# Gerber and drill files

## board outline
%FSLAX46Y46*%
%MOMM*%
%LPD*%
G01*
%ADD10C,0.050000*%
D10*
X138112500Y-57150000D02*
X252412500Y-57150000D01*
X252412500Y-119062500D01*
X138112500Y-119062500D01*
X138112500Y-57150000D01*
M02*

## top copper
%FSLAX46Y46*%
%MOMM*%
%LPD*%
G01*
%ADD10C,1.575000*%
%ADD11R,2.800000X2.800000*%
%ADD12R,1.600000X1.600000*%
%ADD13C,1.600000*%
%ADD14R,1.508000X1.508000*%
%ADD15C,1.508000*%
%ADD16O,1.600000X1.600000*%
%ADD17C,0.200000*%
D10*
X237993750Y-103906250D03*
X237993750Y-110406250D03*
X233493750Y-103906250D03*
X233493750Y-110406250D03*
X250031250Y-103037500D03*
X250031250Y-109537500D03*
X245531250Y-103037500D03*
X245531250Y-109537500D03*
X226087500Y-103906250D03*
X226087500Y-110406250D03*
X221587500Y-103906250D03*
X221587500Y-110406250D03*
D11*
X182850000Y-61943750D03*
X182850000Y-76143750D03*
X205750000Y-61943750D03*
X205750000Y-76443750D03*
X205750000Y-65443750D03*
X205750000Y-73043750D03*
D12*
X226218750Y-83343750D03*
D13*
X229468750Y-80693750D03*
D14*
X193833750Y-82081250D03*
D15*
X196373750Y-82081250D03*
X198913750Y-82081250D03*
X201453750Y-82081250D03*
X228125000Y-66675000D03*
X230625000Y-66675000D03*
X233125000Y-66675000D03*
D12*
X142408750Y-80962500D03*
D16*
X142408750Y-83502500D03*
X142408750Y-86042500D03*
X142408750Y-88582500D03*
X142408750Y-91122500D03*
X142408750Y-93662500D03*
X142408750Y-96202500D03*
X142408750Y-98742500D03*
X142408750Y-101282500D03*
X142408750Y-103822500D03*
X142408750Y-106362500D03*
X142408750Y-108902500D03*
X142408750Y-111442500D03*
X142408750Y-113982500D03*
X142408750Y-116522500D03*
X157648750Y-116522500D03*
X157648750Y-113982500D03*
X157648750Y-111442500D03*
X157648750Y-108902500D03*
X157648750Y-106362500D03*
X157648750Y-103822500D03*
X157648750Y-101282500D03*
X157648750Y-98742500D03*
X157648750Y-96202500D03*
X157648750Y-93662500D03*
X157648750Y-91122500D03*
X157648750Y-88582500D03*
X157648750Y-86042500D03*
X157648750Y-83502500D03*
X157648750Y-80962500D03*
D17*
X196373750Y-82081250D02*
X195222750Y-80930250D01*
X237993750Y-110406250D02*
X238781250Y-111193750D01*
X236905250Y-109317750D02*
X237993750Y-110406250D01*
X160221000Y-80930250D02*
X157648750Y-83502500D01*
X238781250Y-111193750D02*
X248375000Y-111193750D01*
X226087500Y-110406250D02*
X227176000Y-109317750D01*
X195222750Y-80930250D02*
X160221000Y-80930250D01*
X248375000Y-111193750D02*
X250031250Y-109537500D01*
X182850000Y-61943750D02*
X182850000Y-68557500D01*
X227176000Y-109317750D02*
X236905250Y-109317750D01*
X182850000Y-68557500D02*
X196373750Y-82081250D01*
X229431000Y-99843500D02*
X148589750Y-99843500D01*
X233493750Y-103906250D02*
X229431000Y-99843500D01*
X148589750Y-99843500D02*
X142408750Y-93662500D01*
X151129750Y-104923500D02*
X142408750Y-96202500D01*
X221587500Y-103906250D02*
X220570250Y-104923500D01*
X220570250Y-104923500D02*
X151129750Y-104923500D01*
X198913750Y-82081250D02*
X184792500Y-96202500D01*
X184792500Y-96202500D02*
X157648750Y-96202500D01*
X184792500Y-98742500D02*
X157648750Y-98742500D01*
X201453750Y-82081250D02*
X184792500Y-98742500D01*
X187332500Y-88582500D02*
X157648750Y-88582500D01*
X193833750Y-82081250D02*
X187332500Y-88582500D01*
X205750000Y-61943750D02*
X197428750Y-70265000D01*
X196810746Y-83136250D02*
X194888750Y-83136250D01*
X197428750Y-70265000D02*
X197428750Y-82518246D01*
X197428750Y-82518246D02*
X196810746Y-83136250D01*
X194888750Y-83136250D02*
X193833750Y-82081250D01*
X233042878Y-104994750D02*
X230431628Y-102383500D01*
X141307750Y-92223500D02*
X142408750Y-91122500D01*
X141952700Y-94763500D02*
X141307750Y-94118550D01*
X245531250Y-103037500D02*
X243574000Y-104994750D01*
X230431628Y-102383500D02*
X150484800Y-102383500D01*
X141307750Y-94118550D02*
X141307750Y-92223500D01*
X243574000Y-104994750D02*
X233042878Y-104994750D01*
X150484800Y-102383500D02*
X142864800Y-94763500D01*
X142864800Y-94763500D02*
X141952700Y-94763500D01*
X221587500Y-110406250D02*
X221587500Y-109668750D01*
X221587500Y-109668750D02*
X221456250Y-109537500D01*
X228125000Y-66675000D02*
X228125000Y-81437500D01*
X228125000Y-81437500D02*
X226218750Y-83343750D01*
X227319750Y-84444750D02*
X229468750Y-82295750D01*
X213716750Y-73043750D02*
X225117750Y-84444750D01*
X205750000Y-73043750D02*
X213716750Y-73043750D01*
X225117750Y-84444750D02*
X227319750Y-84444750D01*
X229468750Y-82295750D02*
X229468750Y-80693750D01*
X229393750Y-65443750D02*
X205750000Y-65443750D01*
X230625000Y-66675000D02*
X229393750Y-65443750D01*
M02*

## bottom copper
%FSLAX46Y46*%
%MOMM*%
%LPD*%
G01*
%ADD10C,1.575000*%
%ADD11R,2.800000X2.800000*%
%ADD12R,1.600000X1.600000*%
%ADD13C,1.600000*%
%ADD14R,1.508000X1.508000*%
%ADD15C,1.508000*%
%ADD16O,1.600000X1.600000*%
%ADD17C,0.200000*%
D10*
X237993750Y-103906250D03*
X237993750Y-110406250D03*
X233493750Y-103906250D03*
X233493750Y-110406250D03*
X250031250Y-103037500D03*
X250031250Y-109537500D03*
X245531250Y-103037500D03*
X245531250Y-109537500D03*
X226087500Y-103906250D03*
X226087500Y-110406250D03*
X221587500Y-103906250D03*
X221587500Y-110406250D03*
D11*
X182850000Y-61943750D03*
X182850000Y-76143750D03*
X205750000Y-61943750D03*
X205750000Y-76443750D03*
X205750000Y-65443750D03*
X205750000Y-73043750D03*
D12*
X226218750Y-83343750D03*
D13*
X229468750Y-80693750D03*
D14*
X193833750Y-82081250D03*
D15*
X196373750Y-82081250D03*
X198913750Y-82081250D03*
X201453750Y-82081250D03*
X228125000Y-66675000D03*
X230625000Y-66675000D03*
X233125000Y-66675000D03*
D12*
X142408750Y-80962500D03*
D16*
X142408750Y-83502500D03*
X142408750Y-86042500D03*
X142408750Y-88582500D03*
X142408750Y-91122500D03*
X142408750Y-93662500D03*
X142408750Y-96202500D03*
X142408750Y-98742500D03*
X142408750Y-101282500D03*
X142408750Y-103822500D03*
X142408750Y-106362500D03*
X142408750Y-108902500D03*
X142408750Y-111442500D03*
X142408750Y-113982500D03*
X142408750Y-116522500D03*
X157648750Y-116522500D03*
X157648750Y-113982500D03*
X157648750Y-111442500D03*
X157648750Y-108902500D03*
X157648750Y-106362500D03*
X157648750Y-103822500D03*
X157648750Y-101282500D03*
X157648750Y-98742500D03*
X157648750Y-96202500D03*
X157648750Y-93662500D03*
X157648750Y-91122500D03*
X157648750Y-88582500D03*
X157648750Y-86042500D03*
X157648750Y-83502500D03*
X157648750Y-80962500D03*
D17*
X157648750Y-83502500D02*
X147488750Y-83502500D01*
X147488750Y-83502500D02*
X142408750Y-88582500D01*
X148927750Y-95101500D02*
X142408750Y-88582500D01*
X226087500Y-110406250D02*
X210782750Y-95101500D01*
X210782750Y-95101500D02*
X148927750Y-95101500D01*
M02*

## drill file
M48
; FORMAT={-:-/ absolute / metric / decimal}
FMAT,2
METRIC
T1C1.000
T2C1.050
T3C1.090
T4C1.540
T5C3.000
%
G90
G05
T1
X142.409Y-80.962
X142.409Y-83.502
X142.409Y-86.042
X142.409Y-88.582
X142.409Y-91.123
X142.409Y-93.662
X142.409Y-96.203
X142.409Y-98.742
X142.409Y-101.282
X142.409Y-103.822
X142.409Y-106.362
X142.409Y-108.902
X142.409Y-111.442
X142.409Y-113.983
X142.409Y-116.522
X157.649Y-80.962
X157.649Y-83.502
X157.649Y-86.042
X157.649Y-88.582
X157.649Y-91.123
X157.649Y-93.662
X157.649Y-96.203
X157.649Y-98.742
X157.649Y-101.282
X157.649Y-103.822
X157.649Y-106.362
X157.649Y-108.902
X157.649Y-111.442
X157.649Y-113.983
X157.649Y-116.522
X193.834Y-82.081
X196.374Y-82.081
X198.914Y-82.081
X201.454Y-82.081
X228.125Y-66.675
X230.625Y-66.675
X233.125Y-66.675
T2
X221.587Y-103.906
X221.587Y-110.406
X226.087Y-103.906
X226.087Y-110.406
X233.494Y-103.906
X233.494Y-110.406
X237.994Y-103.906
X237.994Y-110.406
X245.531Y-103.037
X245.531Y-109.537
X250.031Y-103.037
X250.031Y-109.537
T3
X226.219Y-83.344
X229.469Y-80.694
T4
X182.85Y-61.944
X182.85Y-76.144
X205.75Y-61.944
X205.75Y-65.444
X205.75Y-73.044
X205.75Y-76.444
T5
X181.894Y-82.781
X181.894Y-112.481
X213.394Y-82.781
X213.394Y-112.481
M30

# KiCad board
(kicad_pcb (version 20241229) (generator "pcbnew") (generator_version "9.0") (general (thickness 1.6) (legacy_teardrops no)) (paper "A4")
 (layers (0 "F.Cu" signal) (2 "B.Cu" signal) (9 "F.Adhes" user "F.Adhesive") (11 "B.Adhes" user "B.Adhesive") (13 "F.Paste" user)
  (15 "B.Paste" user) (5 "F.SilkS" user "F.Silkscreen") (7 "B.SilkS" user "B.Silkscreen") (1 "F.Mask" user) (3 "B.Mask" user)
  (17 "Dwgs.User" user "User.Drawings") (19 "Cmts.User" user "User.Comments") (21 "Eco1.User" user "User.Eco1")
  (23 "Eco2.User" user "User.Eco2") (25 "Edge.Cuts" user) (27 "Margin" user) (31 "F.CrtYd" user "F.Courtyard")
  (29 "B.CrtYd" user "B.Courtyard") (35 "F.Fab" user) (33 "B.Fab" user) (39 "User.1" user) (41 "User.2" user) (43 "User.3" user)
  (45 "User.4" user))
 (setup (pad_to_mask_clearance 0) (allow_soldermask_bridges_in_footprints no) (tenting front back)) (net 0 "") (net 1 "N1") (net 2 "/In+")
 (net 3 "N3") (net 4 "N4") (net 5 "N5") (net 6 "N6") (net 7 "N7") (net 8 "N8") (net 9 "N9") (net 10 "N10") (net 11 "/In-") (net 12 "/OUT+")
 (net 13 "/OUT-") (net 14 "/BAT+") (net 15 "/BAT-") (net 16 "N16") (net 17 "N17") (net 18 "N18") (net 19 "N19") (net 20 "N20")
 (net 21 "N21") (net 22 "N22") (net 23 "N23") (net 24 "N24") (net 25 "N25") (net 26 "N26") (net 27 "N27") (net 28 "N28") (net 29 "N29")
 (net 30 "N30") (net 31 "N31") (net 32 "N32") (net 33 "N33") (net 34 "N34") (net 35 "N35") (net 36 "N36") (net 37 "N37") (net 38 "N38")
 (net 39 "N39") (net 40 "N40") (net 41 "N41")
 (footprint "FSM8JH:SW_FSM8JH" (layer "F.Cu") (at 235.74375 107.15625)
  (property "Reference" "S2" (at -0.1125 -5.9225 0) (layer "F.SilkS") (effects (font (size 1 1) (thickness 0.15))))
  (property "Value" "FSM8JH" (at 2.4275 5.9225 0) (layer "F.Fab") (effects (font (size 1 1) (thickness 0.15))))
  (pad "1" thru_hole circle (at 2.25 -3.25) (size 1.575 1.575) (drill 1.05) (layers "*.Cu" "*.Mask") (remove_unused_layers no) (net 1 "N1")
   (solder_mask_margin 0.102))
  (pad "2" thru_hole circle (at 2.25 3.25) (size 1.575 1.575) (drill 1.05) (layers "*.Cu" "*.Mask") (remove_unused_layers no) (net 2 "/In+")
   (solder_mask_margin 0.102))
  (pad "3" thru_hole circle (at -2.25 -3.25) (size 1.575 1.575) (drill 1.05) (layers "*.Cu" "*.Mask") (remove_unused_layers no) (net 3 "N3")
   (solder_mask_margin 0.102))
  (pad "4" thru_hole circle (at -2.25 3.25) (size 1.575 1.575) (drill 1.05) (layers "*.Cu" "*.Mask") (remove_unused_layers no) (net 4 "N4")
   (solder_mask_margin 0.102)))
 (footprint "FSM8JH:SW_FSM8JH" (layer "F.Cu") (at 247.78125 106.2875)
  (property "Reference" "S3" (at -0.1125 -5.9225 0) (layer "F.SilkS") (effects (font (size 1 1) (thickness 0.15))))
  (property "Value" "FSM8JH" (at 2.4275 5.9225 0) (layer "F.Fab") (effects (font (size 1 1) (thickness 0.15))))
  (pad "1" thru_hole circle (at 2.25 -3.25) (size 1.575 1.575) (drill 1.05) (layers "*.Cu" "*.Mask") (remove_unused_layers no) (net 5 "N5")
   (solder_mask_margin 0.102))
  (pad "2" thru_hole circle (at 2.25 3.25) (size 1.575 1.575) (drill 1.05) (layers "*.Cu" "*.Mask") (remove_unused_layers no) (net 2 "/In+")
   (solder_mask_margin 0.102))
  (pad "3" thru_hole circle (at -2.25 -3.25) (size 1.575 1.575) (drill 1.05) (layers "*.Cu" "*.Mask") (remove_unused_layers no) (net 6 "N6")
   (solder_mask_margin 0.102))
  (pad "4" thru_hole circle (at -2.25 3.25) (size 1.575 1.575) (drill 1.05) (layers "*.Cu" "*.Mask") (remove_unused_layers no) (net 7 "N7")
   (solder_mask_margin 0.102)))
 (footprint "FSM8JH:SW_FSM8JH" (layer "F.Cu") (at 223.8375 107.15625)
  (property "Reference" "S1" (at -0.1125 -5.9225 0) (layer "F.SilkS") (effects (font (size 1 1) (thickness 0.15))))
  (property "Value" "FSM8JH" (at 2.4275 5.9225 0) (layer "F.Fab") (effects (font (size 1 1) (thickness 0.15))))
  (pad "1" thru_hole circle (at 2.25 -3.25) (size 1.575 1.575) (drill 1.05) (layers "*.Cu" "*.Mask") (remove_unused_layers no) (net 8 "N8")
   (solder_mask_margin 0.102))
  (pad "2" thru_hole circle (at 2.25 3.25) (size 1.575 1.575) (drill 1.05) (layers "*.Cu" "*.Mask") (remove_unused_layers no) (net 2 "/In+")
   (solder_mask_margin 0.102))
  (pad "3" thru_hole circle (at -2.25 -3.25) (size 1.575 1.575) (drill 1.05) (layers "*.Cu" "*.Mask") (remove_unused_layers no) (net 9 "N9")
   (solder_mask_margin 0.102))
  (pad "4" thru_hole circle (at -2.25 3.25) (size 1.575 1.575) (drill 1.05) (layers "*.Cu" "*.Mask") (remove_unused_layers no)
   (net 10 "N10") (solder_mask_margin 0.102)))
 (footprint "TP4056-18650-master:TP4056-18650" (layer "F.Cu") (at 181.15 60.24375)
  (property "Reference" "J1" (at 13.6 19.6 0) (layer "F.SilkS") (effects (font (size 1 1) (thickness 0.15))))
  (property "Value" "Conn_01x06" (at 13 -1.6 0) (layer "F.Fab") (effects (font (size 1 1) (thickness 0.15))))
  (pad "1" thru_hole rect (at 1.7 1.7) (size 2.8 2.8) (drill 1.54) (layers "*.Cu" "*.Mask") (remove_unused_layers no) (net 2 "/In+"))
  (pad "2" thru_hole rect (at 1.7 15.9) (size 2.8 2.8) (drill 1.54) (layers "*.Cu" "*.Mask") (remove_unused_layers no) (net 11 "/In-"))
  (pad "3" thru_hole rect (at 24.6 1.7) (size 2.8 2.8) (drill 1.54) (layers "*.Cu" "*.Mask") (remove_unused_layers no) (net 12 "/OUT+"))
  (pad "4" thru_hole rect (at 24.6 16.2) (size 2.8 2.8) (drill 1.54) (layers "*.Cu" "*.Mask") (remove_unused_layers no) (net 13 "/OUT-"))
  (pad "5" thru_hole rect (at 24.6 5.2) (size 2.8 2.8) (drill 1.54) (layers "*.Cu" "*.Mask") (remove_unused_layers no) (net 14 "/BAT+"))
  (pad "6" thru_hole rect (at 24.6 12.8) (size 2.8 2.8) (drill 1.54) (layers "*.Cu" "*.Mask") (remove_unused_layers no) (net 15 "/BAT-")))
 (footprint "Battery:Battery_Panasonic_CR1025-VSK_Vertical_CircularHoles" (layer "F.Cu") (at 226.21875 83.34375)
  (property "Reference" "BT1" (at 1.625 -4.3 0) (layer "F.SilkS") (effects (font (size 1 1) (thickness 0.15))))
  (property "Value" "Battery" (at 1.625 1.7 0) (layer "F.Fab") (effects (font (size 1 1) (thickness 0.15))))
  (pad "1" thru_hole rect (at 0 0) (size 1.6 1.6) (drill 1.09) (layers "*.Cu" "*.Mask") (remove_unused_layers no) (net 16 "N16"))
  (pad "2" thru_hole circle (at 3.25 -2.65) (size 1.6 1.6) (drill 1.09) (layers "*.Cu" "*.Mask") (remove_unused_layers no) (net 15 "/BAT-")))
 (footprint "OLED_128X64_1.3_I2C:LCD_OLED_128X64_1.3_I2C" (layer "F.Cu") (at 197.64375 97.63125)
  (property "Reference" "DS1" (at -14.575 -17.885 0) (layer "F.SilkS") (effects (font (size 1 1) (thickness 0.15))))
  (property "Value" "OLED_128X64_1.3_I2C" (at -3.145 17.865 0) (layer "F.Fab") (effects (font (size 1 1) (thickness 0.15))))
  (pad "" np_thru_hole circle (at -15.75 -14.85) (size 3 3) (drill 3) (layers "*.Cu" "*.Mask"))
  (pad "" np_thru_hole circle (at -15.75 14.85) (size 3 3) (drill 3) (layers "*.Cu" "*.Mask"))
  (pad "" np_thru_hole circle (at 15.75 -14.85) (size 3 3) (drill 3) (layers "*.Cu" "*.Mask"))
  (pad "" np_thru_hole circle (at 15.75 14.85) (size 3 3) (drill 3) (layers "*.Cu" "*.Mask"))
  (pad "1" thru_hole rect (at -3.81 -15.55) (size 1.508 1.508) (drill 1) (layers "*.Cu" "*.Mask") (remove_unused_layers no) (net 12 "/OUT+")
   (solder_mask_margin 0.102))
  (pad "2" thru_hole circle (at -1.27 -15.55) (size 1.508 1.508) (drill 1) (layers "*.Cu" "*.Mask") (remove_unused_layers no) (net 2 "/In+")
   (solder_mask_margin 0.102))
  (pad "3" thru_hole circle (at 1.27 -15.55) (size 1.508 1.508) (drill 1) (layers "*.Cu" "*.Mask") (remove_unused_layers no) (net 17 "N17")
   (solder_mask_margin 0.102))
  (pad "4" thru_hole circle (at 3.81 -15.55) (size 1.508 1.508) (drill 1) (layers "*.Cu" "*.Mask") (remove_unused_layers no) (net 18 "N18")
   (solder_mask_margin 0.102)))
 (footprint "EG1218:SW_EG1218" (layer "F.Cu") (at 230.625 66.675)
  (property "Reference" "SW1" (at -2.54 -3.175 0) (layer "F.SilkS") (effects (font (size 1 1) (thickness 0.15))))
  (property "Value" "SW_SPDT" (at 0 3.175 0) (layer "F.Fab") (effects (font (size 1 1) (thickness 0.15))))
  (pad "1" thru_hole circle (at -2.5 0) (size 1.508 1.508) (drill 1) (layers "*.Cu" "*.Mask") (remove_unused_layers no) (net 16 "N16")
   (solder_mask_margin 0.102))
  (pad "2" thru_hole circle (at 0 0) (size 1.508 1.508) (drill 1) (layers "*.Cu" "*.Mask") (remove_unused_layers no) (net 14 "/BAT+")
   (solder_mask_margin 0.102))
  (pad "3" thru_hole circle (at 2.5 0) (size 1.508 1.508) (drill 1) (layers "*.Cu" "*.Mask") (remove_unused_layers no) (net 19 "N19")
   (solder_mask_margin 0.102)))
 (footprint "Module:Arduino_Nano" (layer "F.Cu") (at 142.40875 80.9625)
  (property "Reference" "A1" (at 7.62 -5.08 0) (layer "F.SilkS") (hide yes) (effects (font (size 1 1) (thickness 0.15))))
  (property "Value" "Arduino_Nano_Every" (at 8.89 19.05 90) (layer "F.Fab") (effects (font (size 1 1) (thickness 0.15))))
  (pad "1" thru_hole rect (at 0 0) (size 1.6 1.6) (drill 1) (layers "*.Cu" "*.Mask") (remove_unused_layers no) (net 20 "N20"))
  (pad "2" thru_hole oval (at 0 2.54) (size 1.6 1.6) (drill 1) (layers "*.Cu" "*.Mask") (remove_unused_layers no) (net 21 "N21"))
  (pad "3" thru_hole oval (at 0 5.08) (size 1.6 1.6) (drill 1) (layers "*.Cu" "*.Mask") (remove_unused_layers no) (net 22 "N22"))
  (pad "4" thru_hole oval (at 0 7.62) (size 1.6 1.6) (drill 1) (layers "*.Cu" "*.Mask") (remove_unused_layers no) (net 2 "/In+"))
  (pad "5" thru_hole oval (at 0 10.16) (size 1.6 1.6) (drill 1) (layers "*.Cu" "*.Mask") (remove_unused_layers no) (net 6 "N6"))
  (pad "6" thru_hole oval (at 0 12.7) (size 1.6 1.6) (drill 1) (layers "*.Cu" "*.Mask") (remove_unused_layers no) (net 3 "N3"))
  (pad "7" thru_hole oval (at 0 15.24) (size 1.6 1.6) (drill 1) (layers "*.Cu" "*.Mask") (remove_unused_layers no) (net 9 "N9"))
  (pad "8" thru_hole oval (at 0 17.78) (size 1.6 1.6) (drill 1) (layers "*.Cu" "*.Mask") (remove_unused_layers no) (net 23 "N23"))
  (pad "9" thru_hole oval (at 0 20.32) (size 1.6 1.6) (drill 1) (layers "*.Cu" "*.Mask") (remove_unused_layers no) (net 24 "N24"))
  (pad "10" thru_hole oval (at 0 22.86) (size 1.6 1.6) (drill 1) (layers "*.Cu" "*.Mask") (remove_unused_layers no) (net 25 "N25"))
  (pad "11" thru_hole oval (at 0 25.4) (size 1.6 1.6) (drill 1) (layers "*.Cu" "*.Mask") (remove_unused_layers no) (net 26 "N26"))
  (pad "12" thru_hole oval (at 0 27.94) (size 1.6 1.6) (drill 1) (layers "*.Cu" "*.Mask") (remove_unused_layers no) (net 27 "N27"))
  (pad "13" thru_hole oval (at 0 30.48) (size 1.6 1.6) (drill 1) (layers "*.Cu" "*.Mask") (remove_unused_layers no) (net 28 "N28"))
  (pad "14" thru_hole oval (at 0 33.02) (size 1.6 1.6) (drill 1) (layers "*.Cu" "*.Mask") (remove_unused_layers no) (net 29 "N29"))
  (pad "15" thru_hole oval (at 0 35.56) (size 1.6 1.6) (drill 1) (layers "*.Cu" "*.Mask") (remove_unused_layers no) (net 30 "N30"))
  (pad "16" thru_hole oval (at 15.24 35.56) (size 1.6 1.6) (drill 1) (layers "*.Cu" "*.Mask") (remove_unused_layers no) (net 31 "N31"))
  (pad "17" thru_hole oval (at 15.24 33.02) (size 1.6 1.6) (drill 1) (layers "*.Cu" "*.Mask") (remove_unused_layers no) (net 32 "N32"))
  (pad "18" thru_hole oval (at 15.24 30.48) (size 1.6 1.6) (drill 1) (layers "*.Cu" "*.Mask") (remove_unused_layers no) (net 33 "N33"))
  (pad "19" thru_hole oval (at 15.24 27.94) (size 1.6 1.6) (drill 1) (layers "*.Cu" "*.Mask") (remove_unused_layers no) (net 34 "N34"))
  (pad "20" thru_hole oval (at 15.24 25.4) (size 1.6 1.6) (drill 1) (layers "*.Cu" "*.Mask") (remove_unused_layers no) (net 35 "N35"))
  (pad "21" thru_hole oval (at 15.24 22.86) (size 1.6 1.6) (drill 1) (layers "*.Cu" "*.Mask") (remove_unused_layers no) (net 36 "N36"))
  (pad "22" thru_hole oval (at 15.24 20.32) (size 1.6 1.6) (drill 1) (layers "*.Cu" "*.Mask") (remove_unused_layers no) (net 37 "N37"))
  (pad "23" thru_hole oval (at 15.24 17.78) (size 1.6 1.6) (drill 1) (layers "*.Cu" "*.Mask") (remove_unused_layers no) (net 18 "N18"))
  (pad "24" thru_hole oval (at 15.24 15.24) (size 1.6 1.6) (drill 1) (layers "*.Cu" "*.Mask") (remove_unused_layers no) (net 17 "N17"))
  (pad "25" thru_hole oval (at 15.24 12.7) (size 1.6 1.6) (drill 1) (layers "*.Cu" "*.Mask") (remove_unused_layers no) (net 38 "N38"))
  (pad "26" thru_hole oval (at 15.24 10.16) (size 1.6 1.6) (drill 1) (layers "*.Cu" "*.Mask") (remove_unused_layers no) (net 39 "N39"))
  (pad "27" thru_hole oval (at 15.24 7.62) (size 1.6 1.6) (drill 1) (layers "*.Cu" "*.Mask") (remove_unused_layers no) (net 12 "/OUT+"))
  (pad "28" thru_hole oval (at 15.24 5.08) (size 1.6 1.6) (drill 1) (layers "*.Cu" "*.Mask") (remove_unused_layers no) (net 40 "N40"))
  (pad "29" thru_hole oval (at 15.24 2.54) (size 1.6 1.6) (drill 1) (layers "*.Cu" "*.Mask") (remove_unused_layers no) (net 2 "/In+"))
  (pad "30" thru_hole oval (at 15.24 0) (size 1.6 1.6) (drill 1) (layers "*.Cu" "*.Mask") (remove_unused_layers no) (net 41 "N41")))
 (gr_rect (start 138.1125 57.15) (end 252.4125 119.0625) (stroke (width 0.05) (type default)) (fill no) (layer "Edge.Cuts"))
 (segment (start 196.37375 82.08125) (end 195.22275 80.93025) (width 0.2) (layer "F.Cu") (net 2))
 (segment (start 237.99375 110.40625) (end 238.78125 111.19375) (width 0.2) (layer "F.Cu") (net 2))
 (segment (start 236.90525 109.31775) (end 237.99375 110.40625) (width 0.2) (layer "F.Cu") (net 2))
 (segment (start 160.221 80.93025) (end 157.64875 83.5025) (width 0.2) (layer "F.Cu") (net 2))
 (segment (start 238.78125 111.19375) (end 248.375 111.19375) (width 0.2) (layer "F.Cu") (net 2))
 (segment (start 226.0875 110.40625) (end 227.176 109.31775) (width 0.2) (layer "F.Cu") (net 2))
 (segment (start 195.22275 80.93025) (end 160.221 80.93025) (width 0.2) (layer "F.Cu") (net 2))
 (segment (start 248.375 111.19375) (end 250.03125 109.5375) (width 0.2) (layer "F.Cu") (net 2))
 (segment (start 182.85 61.94375) (end 182.85 68.5575) (width 0.2) (layer "F.Cu") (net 2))
 (segment (start 227.176 109.31775) (end 236.90525 109.31775) (width 0.2) (layer "F.Cu") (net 2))
 (segment (start 182.85 68.5575) (end 196.37375 82.08125) (width 0.2) (layer "F.Cu") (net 2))
 (segment (start 157.64875 83.5025) (end 147.48875 83.5025) (width 0.2) (layer "B.Cu") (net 2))
 (segment (start 147.48875 83.5025) (end 142.40875 88.5825) (width 0.2) (layer "B.Cu") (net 2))
 (segment (start 148.92775 95.1015) (end 142.40875 88.5825) (width 0.2) (layer "B.Cu") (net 2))
 (segment (start 226.0875 110.40625) (end 210.78275 95.1015) (width 0.2) (layer "B.Cu") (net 2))
 (segment (start 210.78275 95.1015) (end 148.92775 95.1015) (width 0.2) (layer "B.Cu") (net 2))
 (segment (start 229.431 99.8435) (end 148.58975 99.8435) (width 0.2) (layer "F.Cu") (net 3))
 (segment (start 233.49375 103.90625) (end 229.431 99.8435) (width 0.2) (layer "F.Cu") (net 3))
 (segment (start 148.58975 99.8435) (end 142.40875 93.6625) (width 0.2) (layer "F.Cu") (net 3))
 (segment (start 151.12975 104.9235) (end 142.40875 96.2025) (width 0.2) (layer "F.Cu") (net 9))
 (segment (start 221.5875 103.90625) (end 220.57025 104.9235) (width 0.2) (layer "F.Cu") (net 9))
 (segment (start 220.57025 104.9235) (end 151.12975 104.9235) (width 0.2) (layer "F.Cu") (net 9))
 (segment (start 198.91375 82.08125) (end 184.7925 96.2025) (width 0.2) (layer "F.Cu") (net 17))
 (segment (start 184.7925 96.2025) (end 157.64875 96.2025) (width 0.2) (layer "F.Cu") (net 17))
 (segment (start 184.7925 98.7425) (end 157.64875 98.7425) (width 0.2) (layer "F.Cu") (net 18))
 (segment (start 201.45375 82.08125) (end 184.7925 98.7425) (width 0.2) (layer "F.Cu") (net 18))
 (segment (start 187.3325 88.5825) (end 157.64875 88.5825) (width 0.2) (layer "F.Cu") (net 12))
 (segment (start 193.83375 82.08125) (end 187.3325 88.5825) (width 0.2) (layer "F.Cu") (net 12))
 (segment (start 205.75 61.94375) (end 197.42875 70.265) (width 0.2) (layer "F.Cu") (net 12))
 (segment (start 196.810746 83.13625) (end 194.88875 83.13625) (width 0.2) (layer "F.Cu") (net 12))
 (segment (start 197.42875 70.265) (end 197.42875 82.518246) (width 0.2) (layer "F.Cu") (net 12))
 (segment (start 197.42875 82.518246) (end 196.810746 83.13625) (width 0.2) (layer "F.Cu") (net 12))
 (segment (start 194.88875 83.13625) (end 193.83375 82.08125) (width 0.2) (layer "F.Cu") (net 12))
 (segment (start 233.042878 104.99475) (end 230.431628 102.3835) (width 0.2) (layer "F.Cu") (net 6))
 (segment (start 141.30775 92.2235) (end 142.40875 91.1225) (width 0.2) (layer "F.Cu") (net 6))
 (segment (start 141.9527 94.7635) (end 141.30775 94.11855) (width 0.2) (layer "F.Cu") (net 6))
 (segment (start 245.53125 103.0375) (end 243.574 104.99475) (width 0.2) (layer "F.Cu") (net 6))
 (segment (start 230.431628 102.3835) (end 150.4848 102.3835) (width 0.2) (layer "F.Cu") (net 6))
 (segment (start 141.30775 94.11855) (end 141.30775 92.2235) (width 0.2) (layer "F.Cu") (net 6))
 (segment (start 243.574 104.99475) (end 233.042878 104.99475) (width 0.2) (layer "F.Cu") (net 6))
 (segment (start 150.4848 102.3835) (end 142.8648 94.7635) (width 0.2) (layer "F.Cu") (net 6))
 (segment (start 142.8648 94.7635) (end 141.9527 94.7635) (width 0.2) (layer "F.Cu") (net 6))
 (segment (start 221.5875 110.40625) (end 221.5875 109.66875) (width 0.2) (layer "F.Cu") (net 10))
 (segment (start 221.5875 109.66875) (end 221.45625 109.5375) (width 0.2) (layer "F.Cu") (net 10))
 (segment (start 228.125 66.675) (end 228.125 81.4375) (width 0.2) (layer "F.Cu") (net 16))
 (segment (start 228.125 81.4375) (end 226.21875 83.34375) (width 0.2) (layer "F.Cu") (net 16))
 (segment (start 227.31975 84.44475) (end 229.46875 82.29575) (width 0.2) (layer "F.Cu") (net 15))
 (segment (start 213.71675 73.04375) (end 225.11775 84.44475) (width 0.2) (layer "F.Cu") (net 15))
 (segment (start 205.75 73.04375) (end 213.71675 73.04375) (width 0.2) (layer "F.Cu") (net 15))
 (segment (start 225.11775 84.44475) (end 227.31975 84.44475) (width 0.2) (layer "F.Cu") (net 15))
 (segment (start 229.46875 82.29575) (end 229.46875 80.69375) (width 0.2) (layer "F.Cu") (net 15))
 (segment (start 229.39375 65.44375) (end 205.75 65.44375) (width 0.2) (layer "F.Cu") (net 14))
 (segment (start 230.625 66.675) (end 229.39375 65.44375) (width 0.2) (layer "F.Cu") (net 14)))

